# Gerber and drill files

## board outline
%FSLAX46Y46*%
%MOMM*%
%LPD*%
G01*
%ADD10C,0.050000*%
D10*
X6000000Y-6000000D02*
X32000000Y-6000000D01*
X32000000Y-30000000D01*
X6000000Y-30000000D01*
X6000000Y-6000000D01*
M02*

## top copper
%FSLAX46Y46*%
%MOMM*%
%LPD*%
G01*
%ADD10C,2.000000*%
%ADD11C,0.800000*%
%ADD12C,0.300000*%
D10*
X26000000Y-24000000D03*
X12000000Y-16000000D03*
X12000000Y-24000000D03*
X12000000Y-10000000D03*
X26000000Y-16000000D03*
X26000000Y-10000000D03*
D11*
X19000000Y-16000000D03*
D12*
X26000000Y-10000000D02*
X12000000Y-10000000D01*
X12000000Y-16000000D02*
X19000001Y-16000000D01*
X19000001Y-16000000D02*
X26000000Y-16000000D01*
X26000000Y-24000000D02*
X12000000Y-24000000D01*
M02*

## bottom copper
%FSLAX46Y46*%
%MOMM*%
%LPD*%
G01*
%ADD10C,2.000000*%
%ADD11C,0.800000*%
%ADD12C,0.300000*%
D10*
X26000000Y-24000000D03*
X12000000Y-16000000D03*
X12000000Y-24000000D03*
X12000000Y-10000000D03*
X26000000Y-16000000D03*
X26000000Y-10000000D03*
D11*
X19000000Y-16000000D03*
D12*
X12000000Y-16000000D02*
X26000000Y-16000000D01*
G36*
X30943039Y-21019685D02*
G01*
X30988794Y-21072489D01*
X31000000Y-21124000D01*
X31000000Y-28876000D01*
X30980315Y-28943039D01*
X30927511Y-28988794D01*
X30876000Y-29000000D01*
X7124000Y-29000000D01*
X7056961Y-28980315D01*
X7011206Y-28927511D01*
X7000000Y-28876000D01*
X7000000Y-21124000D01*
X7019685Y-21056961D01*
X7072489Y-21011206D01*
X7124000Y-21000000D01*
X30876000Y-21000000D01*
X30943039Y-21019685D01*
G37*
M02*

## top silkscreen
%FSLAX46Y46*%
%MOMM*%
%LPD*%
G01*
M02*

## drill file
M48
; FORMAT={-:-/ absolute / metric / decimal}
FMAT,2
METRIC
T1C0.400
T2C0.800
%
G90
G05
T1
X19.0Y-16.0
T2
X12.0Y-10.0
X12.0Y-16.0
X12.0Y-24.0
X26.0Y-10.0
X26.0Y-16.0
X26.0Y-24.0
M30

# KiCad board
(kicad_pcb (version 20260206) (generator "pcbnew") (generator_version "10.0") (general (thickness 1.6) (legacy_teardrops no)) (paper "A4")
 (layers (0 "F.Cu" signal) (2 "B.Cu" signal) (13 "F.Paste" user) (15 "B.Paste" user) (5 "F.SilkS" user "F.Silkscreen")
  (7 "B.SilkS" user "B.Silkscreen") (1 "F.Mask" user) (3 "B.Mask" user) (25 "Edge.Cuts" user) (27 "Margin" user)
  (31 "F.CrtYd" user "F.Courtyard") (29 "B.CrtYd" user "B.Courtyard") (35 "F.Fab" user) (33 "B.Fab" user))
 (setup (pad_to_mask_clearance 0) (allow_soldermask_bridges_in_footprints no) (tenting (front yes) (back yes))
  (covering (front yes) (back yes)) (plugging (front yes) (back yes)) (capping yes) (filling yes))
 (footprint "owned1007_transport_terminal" (layer "F.Cu") (at 26 24)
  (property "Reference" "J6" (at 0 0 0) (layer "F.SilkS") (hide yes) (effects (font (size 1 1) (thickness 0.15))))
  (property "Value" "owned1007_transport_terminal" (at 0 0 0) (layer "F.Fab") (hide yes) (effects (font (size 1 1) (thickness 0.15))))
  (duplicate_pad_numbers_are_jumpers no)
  (pad "1" thru_hole circle (at 0 0) (size 2 2) (drill 0.8) (layers "*.Cu" "*.Mask") (remove_unused_layers no) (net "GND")))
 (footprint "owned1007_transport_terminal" (layer "F.Cu") (at 12 16)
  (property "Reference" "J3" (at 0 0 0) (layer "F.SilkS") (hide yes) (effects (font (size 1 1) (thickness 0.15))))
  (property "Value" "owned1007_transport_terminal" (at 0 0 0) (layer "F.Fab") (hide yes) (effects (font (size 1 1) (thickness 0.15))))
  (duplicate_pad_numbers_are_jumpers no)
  (pad "1" thru_hole circle (at 0 0) (size 2 2) (drill 0.8) (layers "*.Cu" "*.Mask") (remove_unused_layers no) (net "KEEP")))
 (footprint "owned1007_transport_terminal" (layer "F.Cu") (at 12 24)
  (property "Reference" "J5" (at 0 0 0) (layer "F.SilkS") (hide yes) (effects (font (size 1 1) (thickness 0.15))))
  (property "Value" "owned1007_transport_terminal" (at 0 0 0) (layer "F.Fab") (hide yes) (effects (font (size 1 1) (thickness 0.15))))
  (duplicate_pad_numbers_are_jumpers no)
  (pad "1" thru_hole circle (at 0 0) (size 2 2) (drill 0.8) (layers "*.Cu" "*.Mask") (remove_unused_layers no) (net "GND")))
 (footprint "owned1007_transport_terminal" (layer "F.Cu") (at 12 10)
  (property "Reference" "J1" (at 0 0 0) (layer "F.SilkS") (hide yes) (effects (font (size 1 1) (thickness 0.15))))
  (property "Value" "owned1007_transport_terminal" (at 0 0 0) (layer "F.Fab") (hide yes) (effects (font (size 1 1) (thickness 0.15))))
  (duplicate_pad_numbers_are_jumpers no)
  (pad "1" thru_hole circle (at 0 0) (size 2 2) (drill 0.8) (layers "*.Cu" "*.Mask") (remove_unused_layers no) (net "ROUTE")))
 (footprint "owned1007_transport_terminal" (layer "F.Cu") (at 26 16)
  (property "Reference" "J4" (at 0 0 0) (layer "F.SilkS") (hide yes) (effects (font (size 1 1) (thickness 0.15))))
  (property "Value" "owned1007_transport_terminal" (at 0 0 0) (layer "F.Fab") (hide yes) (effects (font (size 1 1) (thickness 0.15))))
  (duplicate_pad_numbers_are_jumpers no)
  (pad "1" thru_hole circle (at 0 0) (size 2 2) (drill 0.8) (layers "*.Cu" "*.Mask") (remove_unused_layers no) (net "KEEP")))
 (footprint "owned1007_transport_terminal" (layer "F.Cu") (at 26 10)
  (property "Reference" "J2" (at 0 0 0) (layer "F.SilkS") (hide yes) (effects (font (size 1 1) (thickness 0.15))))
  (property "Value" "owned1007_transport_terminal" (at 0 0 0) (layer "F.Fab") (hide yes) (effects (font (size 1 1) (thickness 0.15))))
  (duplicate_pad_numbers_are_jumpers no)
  (pad "1" thru_hole circle (at 0 0) (size 2 2) (drill 0.8) (layers "*.Cu" "*.Mask") (remove_unused_layers no) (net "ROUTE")))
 (gr_rect (start 6 6) (end 32 30) (stroke (width 0.05) (type default)) (fill no) (layer "Edge.Cuts"))
 (segment (start 26 10) (end 12 10) (width 0.3) (layer "F.Cu") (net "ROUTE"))
 (segment (start 12 16) (end 19.000001 16) (width 0.3) (layer "F.Cu") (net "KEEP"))
 (segment (start 19.000001 16) (end 26 16) (width 0.3) (layer "F.Cu") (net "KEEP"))
 (via (at 19 16) (size 0.8) (drill 0.4) (layers "F.Cu" "B.Cu") (capping no) (covering (front no) (back no)) (plugging (front no) (back no))
  (filling no) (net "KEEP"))
 (segment (start 12 16) (end 26 16) (width 0.3) (layer "B.Cu") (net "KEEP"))
 (segment (start 26 24) (end 12 24) (width 0.3) (layer "F.Cu") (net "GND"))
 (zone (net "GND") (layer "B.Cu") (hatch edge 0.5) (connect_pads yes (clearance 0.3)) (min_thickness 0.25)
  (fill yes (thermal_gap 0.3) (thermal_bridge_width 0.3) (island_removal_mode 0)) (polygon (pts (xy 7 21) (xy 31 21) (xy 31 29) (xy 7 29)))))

